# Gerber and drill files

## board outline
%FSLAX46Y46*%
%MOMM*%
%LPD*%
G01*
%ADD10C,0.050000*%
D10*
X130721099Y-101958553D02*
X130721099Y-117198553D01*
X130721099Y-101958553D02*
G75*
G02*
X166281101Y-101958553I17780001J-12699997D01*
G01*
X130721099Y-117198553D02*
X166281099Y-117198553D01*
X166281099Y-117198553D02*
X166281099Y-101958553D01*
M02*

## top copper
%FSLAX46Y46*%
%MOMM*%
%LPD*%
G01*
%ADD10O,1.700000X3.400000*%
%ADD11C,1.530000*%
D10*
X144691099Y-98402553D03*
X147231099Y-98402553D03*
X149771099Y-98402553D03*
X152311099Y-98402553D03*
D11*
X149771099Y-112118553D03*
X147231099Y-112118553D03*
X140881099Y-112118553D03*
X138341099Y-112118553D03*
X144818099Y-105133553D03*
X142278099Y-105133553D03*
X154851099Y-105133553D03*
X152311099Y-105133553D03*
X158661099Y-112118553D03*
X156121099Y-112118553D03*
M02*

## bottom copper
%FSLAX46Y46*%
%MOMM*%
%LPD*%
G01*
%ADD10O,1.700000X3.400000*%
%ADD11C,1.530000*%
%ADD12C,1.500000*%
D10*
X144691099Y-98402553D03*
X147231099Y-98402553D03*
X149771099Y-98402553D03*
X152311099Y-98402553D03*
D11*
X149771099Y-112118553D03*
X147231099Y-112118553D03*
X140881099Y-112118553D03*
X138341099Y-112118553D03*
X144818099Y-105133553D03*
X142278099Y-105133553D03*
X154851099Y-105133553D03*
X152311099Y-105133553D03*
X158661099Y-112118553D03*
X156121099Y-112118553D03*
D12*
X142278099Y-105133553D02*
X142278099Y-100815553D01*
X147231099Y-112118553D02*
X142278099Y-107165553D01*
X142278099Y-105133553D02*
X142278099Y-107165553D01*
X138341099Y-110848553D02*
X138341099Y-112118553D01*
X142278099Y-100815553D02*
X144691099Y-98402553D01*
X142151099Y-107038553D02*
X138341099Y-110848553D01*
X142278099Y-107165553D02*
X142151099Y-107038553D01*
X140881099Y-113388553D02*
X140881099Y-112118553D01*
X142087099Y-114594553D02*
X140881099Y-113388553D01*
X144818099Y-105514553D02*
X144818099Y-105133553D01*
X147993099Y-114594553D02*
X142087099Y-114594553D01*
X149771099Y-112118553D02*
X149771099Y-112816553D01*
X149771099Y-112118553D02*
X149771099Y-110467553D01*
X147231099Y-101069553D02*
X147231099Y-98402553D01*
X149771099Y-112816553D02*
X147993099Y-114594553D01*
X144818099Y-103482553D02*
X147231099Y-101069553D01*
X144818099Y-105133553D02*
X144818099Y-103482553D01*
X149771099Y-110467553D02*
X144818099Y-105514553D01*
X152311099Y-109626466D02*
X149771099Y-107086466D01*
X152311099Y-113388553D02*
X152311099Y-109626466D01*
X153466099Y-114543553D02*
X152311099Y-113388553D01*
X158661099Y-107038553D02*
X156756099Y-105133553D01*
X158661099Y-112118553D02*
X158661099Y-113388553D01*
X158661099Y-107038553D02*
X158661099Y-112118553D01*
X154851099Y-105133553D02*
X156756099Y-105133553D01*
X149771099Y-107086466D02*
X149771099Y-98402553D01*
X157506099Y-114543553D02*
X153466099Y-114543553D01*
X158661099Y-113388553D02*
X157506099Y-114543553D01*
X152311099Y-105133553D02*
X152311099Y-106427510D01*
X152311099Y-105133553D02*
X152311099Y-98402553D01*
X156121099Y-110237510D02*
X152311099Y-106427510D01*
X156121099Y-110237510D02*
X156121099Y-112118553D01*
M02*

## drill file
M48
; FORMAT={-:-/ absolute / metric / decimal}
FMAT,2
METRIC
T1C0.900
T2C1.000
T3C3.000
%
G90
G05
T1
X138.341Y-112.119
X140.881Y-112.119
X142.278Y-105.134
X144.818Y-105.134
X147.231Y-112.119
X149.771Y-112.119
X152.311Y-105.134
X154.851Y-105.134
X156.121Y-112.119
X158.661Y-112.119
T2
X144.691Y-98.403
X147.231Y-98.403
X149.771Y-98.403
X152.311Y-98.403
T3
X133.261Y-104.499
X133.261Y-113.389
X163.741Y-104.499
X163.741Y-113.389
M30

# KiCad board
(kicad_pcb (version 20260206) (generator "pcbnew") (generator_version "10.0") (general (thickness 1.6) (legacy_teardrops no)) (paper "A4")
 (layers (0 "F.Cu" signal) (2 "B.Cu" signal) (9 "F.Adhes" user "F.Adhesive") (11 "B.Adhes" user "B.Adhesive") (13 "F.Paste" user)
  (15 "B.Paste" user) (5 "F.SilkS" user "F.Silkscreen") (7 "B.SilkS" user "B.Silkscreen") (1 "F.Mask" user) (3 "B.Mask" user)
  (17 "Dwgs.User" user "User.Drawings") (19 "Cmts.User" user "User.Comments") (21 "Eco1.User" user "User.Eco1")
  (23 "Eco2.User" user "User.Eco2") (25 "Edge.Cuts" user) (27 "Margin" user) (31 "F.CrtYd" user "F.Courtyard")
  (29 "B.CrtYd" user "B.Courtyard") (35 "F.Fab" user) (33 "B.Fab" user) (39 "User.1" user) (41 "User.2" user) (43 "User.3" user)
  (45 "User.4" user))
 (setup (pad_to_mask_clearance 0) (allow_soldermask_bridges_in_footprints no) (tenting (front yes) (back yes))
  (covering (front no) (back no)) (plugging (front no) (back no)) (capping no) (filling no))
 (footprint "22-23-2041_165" (layer "F.Cu") (at 148.501099 98.402553)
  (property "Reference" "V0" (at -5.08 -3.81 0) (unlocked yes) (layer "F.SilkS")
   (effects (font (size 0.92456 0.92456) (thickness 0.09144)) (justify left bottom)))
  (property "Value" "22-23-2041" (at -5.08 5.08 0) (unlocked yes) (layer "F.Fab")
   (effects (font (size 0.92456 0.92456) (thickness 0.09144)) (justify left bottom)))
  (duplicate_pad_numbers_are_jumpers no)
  (pad "1" thru_hole oval (at -3.81 0 90) (size 3.4 1.7) (drill 1) (layers "*.Cu" "*.Mask") (remove_unused_layers no) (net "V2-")
   (solder_mask_margin 0.1016) (thermal_bridge_angle 0))
  (pad "2" thru_hole oval (at -1.27 0 90) (size 3.4 1.7) (drill 1) (layers "*.Cu" "*.Mask") (remove_unused_layers no) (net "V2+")
   (solder_mask_margin 0.1016) (thermal_bridge_angle 0))
  (pad "3" thru_hole oval (at 1.27 0 90) (size 3.4 1.7) (drill 1) (layers "*.Cu" "*.Mask") (remove_unused_layers no) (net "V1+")
   (solder_mask_margin 0.1016) (thermal_bridge_angle 0))
  (pad "4" thru_hole oval (at 3.81 0 90) (size 3.4 1.7) (drill 1) (layers "*.Cu" "*.Mask") (remove_unused_layers no) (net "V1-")
   (solder_mask_margin 0.1016) (thermal_bridge_angle 0)))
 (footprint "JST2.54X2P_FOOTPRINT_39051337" (layer "F.Cu") (at 148.501099 112.118553 180)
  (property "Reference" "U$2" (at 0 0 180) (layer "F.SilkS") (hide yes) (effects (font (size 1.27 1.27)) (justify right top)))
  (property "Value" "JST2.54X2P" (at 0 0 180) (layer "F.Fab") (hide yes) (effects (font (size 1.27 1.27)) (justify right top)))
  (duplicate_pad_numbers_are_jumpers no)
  (pad "1" thru_hole circle (at -1.27 0 180) (size 1.53 1.53) (drill 0.9) (layers "*.Cu" "*.Mask") (remove_unused_layers no) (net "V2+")
   (solder_mask_margin 0.1016) (thermal_bridge_angle 0))
  (pad "2" thru_hole circle (at 1.27 0 180) (size 1.53 1.53) (drill 0.9) (layers "*.Cu" "*.Mask") (remove_unused_layers no) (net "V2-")
   (solder_mask_margin 0.1016) (thermal_bridge_angle 0)))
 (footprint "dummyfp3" (layer "F.Cu") (at 133.261099 104.498553)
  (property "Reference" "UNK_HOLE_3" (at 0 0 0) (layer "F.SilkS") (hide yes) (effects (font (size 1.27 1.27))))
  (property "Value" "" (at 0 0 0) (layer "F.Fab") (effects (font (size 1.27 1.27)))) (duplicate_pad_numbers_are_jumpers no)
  (pad "" np_thru_hole circle (at 0 0) (size 3 3) (drill 3) (layers "*.Cu" "*.Mask")))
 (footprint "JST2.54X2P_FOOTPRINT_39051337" (layer "F.Cu") (at 139.611099 112.118553 180)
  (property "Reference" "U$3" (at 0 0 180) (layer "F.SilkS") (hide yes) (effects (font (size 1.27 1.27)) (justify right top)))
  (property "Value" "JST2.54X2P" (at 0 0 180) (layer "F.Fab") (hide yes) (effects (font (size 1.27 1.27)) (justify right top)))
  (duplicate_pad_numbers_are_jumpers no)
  (pad "1" thru_hole circle (at -1.27 0 180) (size 1.53 1.53) (drill 0.9) (layers "*.Cu" "*.Mask") (remove_unused_layers no) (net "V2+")
   (solder_mask_margin 0.1016) (thermal_bridge_angle 0))
  (pad "2" thru_hole circle (at 1.27 0 180) (size 1.53 1.53) (drill 0.9) (layers "*.Cu" "*.Mask") (remove_unused_layers no) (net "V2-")
   (solder_mask_margin 0.1016) (thermal_bridge_angle 0)))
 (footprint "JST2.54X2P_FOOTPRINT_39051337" (layer "F.Cu") (at 143.548099 105.133553 180)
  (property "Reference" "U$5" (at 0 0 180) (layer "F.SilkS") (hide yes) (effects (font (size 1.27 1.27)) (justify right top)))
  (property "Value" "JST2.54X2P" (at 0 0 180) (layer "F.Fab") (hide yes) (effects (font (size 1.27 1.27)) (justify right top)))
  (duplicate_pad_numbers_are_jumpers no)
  (pad "1" thru_hole circle (at -1.27 0 180) (size 1.53 1.53) (drill 0.9) (layers "*.Cu" "*.Mask") (remove_unused_layers no) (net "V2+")
   (solder_mask_margin 0.1016) (thermal_bridge_angle 0))
  (pad "2" thru_hole circle (at 1.27 0 180) (size 1.53 1.53) (drill 0.9) (layers "*.Cu" "*.Mask") (remove_unused_layers no) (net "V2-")
   (solder_mask_margin 0.1016) (thermal_bridge_angle 0)))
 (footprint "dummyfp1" (layer "F.Cu") (at 163.741099 113.388553)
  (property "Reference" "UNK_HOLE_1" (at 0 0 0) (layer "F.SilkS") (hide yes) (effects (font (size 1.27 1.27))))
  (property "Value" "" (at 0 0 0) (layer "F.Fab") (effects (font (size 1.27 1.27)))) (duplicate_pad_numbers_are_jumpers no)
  (pad "" np_thru_hole circle (at 0 0) (size 3 3) (drill 3) (layers "*.Cu" "*.Mask")))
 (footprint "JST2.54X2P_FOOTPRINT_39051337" (layer "F.Cu") (at 153.581099 105.133553 180)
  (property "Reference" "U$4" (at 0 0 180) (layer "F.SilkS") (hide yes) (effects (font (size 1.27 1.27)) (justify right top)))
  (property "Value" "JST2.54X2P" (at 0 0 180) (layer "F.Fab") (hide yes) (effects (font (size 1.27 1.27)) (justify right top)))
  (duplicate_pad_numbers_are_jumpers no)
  (pad "1" thru_hole circle (at -1.27 0 180) (size 1.53 1.53) (drill 0.9) (layers "*.Cu" "*.Mask") (remove_unused_layers no) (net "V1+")
   (solder_mask_margin 0.1016) (thermal_bridge_angle 0))
  (pad "2" thru_hole circle (at 1.27 0 180) (size 1.53 1.53) (drill 0.9) (layers "*.Cu" "*.Mask") (remove_unused_layers no) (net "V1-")
   (solder_mask_margin 0.1016) (thermal_bridge_angle 0)))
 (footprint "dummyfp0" (layer "F.Cu") (at 163.741099 104.498553)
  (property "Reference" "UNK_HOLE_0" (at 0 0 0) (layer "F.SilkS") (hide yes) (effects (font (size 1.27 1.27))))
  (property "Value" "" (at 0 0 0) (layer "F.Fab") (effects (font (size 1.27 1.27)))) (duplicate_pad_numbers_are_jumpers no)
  (pad "" np_thru_hole circle (at 0 0) (size 3 3) (drill 3) (layers "*.Cu" "*.Mask")))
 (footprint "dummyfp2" (layer "F.Cu") (at 133.261099 113.388553)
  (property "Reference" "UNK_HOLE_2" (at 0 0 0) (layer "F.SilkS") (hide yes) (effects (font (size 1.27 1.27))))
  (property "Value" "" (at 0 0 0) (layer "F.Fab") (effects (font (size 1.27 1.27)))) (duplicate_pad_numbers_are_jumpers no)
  (pad "" np_thru_hole circle (at 0 0) (size 3 3) (drill 3) (layers "*.Cu" "*.Mask")))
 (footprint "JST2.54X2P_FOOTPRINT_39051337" (layer "F.Cu") (at 157.391099 112.118553 180)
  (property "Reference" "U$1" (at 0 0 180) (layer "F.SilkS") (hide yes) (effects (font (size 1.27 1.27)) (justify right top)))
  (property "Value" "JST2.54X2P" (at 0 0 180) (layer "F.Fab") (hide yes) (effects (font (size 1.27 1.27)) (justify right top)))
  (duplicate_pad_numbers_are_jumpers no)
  (pad "1" thru_hole circle (at -1.27 0 180) (size 1.53 1.53) (drill 0.9) (layers "*.Cu" "*.Mask") (remove_unused_layers no) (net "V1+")
   (solder_mask_margin 0.1016) (thermal_bridge_angle 0))
  (pad "2" thru_hole circle (at 1.27 0 180) (size 1.53 1.53) (drill 0.9) (layers "*.Cu" "*.Mask") (remove_unused_layers no) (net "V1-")
   (solder_mask_margin 0.1016) (thermal_bridge_angle 0)))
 (gr_line (start 130.721099 101.958553) (end 130.721099 117.198553) (stroke (width 0.05) (type solid)) (layer "Edge.Cuts"))
 (gr_arc (start 130.721099 101.958553) (mid 148.5011 92.808647) (end 166.2811 101.958554) (stroke (width 0.05) (type solid))
  (layer "Edge.Cuts"))
 (gr_line (start 130.721099 117.198553) (end 166.281099 117.198553) (stroke (width 0.05) (type solid)) (layer "Edge.Cuts"))
 (gr_line (start 166.281099 117.198553) (end 166.281099 101.958553) (stroke (width 0.05) (type solid)) (layer "Edge.Cuts"))
 (segment (start 142.278099 105.133553) (end 142.278099 100.815553) (width 1.5) (layer "B.Cu") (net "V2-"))
 (segment (start 147.231099 112.118553) (end 142.278099 107.165553) (width 1.5) (layer "B.Cu") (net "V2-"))
 (segment (start 142.278099 105.133553) (end 142.278099 107.165553) (width 1.5) (layer "B.Cu") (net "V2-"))
 (segment (start 138.341099 110.848553) (end 138.341099 112.118553) (width 1.5) (layer "B.Cu") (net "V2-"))
 (segment (start 142.278099 100.815553) (end 144.691099 98.402553) (width 1.5) (layer "B.Cu") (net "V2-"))
 (segment (start 142.151099 107.038553) (end 138.341099 110.848553) (width 1.5) (layer "B.Cu") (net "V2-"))
 (segment (start 142.278099 107.165553) (end 142.151099 107.038553) (width 1.5) (layer "B.Cu") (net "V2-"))
 (segment (start 140.881099 113.388553) (end 140.881099 112.118553) (width 1.5) (layer "B.Cu") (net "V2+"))
 (segment (start 142.087099 114.594553) (end 140.881099 113.388553) (width 1.5) (layer "B.Cu") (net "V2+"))
 (segment (start 144.818099 105.514553) (end 144.818099 105.133553) (width 1.5) (layer "B.Cu") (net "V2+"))
 (segment (start 147.993099 114.594553) (end 142.087099 114.594553) (width 1.5) (layer "B.Cu") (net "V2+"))
 (segment (start 149.771099 112.118553) (end 149.771099 112.816553) (width 1.5) (layer "B.Cu") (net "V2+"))
 (segment (start 149.771099 112.118553) (end 149.771099 110.467553) (width 1.5) (layer "B.Cu") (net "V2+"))
 (segment (start 147.231099 101.069553) (end 147.231099 98.402553) (width 1.5) (layer "B.Cu") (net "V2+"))
 (segment (start 149.771099 112.816553) (end 147.993099 114.594553) (width 1.5) (layer "B.Cu") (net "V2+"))
 (segment (start 144.818099 103.482553) (end 147.231099 101.069553) (width 1.5) (layer "B.Cu") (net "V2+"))
 (segment (start 144.818099 105.133553) (end 144.818099 103.482553) (width 1.5) (layer "B.Cu") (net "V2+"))
 (segment (start 149.771099 110.467553) (end 144.818099 105.514553) (width 1.5) (layer "B.Cu") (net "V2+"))
 (segment (start 152.311099 109.626466) (end 149.771099 107.086466) (width 1.5) (layer "B.Cu") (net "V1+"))
 (segment (start 152.311099 113.388553) (end 152.311099 109.626466) (width 1.5) (layer "B.Cu") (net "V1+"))
 (segment (start 153.466099 114.543553) (end 152.311099 113.388553) (width 1.5) (layer "B.Cu") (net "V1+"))
 (segment (start 158.661099 107.038553) (end 156.756099 105.133553) (width 1.5) (layer "B.Cu") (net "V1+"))
 (segment (start 158.661099 112.118553) (end 158.661099 113.388553) (width 1.5) (layer "B.Cu") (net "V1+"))
 (segment (start 158.661099 107.038553) (end 158.661099 112.118553) (width 1.5) (layer "B.Cu") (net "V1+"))
 (segment (start 154.851099 105.133553) (end 156.756099 105.133553) (width 1.5) (layer "B.Cu") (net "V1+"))
 (segment (start 149.771099 107.086466) (end 149.771099 98.402553) (width 1.5) (layer "B.Cu") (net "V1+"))
 (segment (start 157.506099 114.543553) (end 153.466099 114.543553) (width 1.5) (layer "B.Cu") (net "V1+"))
 (segment (start 158.661099 113.388553) (end 157.506099 114.543553) (width 1.5) (layer "B.Cu") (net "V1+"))
 (segment (start 152.311099 105.133553) (end 152.311099 106.42751) (width 1.5) (layer "B.Cu") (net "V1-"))
 (segment (start 152.311099 105.133553) (end 152.311099 98.402553) (width 1.5) (layer "B.Cu") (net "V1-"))
 (segment (start 156.121099 110.23751) (end 152.311099 106.42751) (width 1.5) (layer "B.Cu") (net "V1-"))
 (segment (start 156.121099 110.23751) (end 156.121099 112.118553) (width 1.5) (layer "B.Cu") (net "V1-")))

